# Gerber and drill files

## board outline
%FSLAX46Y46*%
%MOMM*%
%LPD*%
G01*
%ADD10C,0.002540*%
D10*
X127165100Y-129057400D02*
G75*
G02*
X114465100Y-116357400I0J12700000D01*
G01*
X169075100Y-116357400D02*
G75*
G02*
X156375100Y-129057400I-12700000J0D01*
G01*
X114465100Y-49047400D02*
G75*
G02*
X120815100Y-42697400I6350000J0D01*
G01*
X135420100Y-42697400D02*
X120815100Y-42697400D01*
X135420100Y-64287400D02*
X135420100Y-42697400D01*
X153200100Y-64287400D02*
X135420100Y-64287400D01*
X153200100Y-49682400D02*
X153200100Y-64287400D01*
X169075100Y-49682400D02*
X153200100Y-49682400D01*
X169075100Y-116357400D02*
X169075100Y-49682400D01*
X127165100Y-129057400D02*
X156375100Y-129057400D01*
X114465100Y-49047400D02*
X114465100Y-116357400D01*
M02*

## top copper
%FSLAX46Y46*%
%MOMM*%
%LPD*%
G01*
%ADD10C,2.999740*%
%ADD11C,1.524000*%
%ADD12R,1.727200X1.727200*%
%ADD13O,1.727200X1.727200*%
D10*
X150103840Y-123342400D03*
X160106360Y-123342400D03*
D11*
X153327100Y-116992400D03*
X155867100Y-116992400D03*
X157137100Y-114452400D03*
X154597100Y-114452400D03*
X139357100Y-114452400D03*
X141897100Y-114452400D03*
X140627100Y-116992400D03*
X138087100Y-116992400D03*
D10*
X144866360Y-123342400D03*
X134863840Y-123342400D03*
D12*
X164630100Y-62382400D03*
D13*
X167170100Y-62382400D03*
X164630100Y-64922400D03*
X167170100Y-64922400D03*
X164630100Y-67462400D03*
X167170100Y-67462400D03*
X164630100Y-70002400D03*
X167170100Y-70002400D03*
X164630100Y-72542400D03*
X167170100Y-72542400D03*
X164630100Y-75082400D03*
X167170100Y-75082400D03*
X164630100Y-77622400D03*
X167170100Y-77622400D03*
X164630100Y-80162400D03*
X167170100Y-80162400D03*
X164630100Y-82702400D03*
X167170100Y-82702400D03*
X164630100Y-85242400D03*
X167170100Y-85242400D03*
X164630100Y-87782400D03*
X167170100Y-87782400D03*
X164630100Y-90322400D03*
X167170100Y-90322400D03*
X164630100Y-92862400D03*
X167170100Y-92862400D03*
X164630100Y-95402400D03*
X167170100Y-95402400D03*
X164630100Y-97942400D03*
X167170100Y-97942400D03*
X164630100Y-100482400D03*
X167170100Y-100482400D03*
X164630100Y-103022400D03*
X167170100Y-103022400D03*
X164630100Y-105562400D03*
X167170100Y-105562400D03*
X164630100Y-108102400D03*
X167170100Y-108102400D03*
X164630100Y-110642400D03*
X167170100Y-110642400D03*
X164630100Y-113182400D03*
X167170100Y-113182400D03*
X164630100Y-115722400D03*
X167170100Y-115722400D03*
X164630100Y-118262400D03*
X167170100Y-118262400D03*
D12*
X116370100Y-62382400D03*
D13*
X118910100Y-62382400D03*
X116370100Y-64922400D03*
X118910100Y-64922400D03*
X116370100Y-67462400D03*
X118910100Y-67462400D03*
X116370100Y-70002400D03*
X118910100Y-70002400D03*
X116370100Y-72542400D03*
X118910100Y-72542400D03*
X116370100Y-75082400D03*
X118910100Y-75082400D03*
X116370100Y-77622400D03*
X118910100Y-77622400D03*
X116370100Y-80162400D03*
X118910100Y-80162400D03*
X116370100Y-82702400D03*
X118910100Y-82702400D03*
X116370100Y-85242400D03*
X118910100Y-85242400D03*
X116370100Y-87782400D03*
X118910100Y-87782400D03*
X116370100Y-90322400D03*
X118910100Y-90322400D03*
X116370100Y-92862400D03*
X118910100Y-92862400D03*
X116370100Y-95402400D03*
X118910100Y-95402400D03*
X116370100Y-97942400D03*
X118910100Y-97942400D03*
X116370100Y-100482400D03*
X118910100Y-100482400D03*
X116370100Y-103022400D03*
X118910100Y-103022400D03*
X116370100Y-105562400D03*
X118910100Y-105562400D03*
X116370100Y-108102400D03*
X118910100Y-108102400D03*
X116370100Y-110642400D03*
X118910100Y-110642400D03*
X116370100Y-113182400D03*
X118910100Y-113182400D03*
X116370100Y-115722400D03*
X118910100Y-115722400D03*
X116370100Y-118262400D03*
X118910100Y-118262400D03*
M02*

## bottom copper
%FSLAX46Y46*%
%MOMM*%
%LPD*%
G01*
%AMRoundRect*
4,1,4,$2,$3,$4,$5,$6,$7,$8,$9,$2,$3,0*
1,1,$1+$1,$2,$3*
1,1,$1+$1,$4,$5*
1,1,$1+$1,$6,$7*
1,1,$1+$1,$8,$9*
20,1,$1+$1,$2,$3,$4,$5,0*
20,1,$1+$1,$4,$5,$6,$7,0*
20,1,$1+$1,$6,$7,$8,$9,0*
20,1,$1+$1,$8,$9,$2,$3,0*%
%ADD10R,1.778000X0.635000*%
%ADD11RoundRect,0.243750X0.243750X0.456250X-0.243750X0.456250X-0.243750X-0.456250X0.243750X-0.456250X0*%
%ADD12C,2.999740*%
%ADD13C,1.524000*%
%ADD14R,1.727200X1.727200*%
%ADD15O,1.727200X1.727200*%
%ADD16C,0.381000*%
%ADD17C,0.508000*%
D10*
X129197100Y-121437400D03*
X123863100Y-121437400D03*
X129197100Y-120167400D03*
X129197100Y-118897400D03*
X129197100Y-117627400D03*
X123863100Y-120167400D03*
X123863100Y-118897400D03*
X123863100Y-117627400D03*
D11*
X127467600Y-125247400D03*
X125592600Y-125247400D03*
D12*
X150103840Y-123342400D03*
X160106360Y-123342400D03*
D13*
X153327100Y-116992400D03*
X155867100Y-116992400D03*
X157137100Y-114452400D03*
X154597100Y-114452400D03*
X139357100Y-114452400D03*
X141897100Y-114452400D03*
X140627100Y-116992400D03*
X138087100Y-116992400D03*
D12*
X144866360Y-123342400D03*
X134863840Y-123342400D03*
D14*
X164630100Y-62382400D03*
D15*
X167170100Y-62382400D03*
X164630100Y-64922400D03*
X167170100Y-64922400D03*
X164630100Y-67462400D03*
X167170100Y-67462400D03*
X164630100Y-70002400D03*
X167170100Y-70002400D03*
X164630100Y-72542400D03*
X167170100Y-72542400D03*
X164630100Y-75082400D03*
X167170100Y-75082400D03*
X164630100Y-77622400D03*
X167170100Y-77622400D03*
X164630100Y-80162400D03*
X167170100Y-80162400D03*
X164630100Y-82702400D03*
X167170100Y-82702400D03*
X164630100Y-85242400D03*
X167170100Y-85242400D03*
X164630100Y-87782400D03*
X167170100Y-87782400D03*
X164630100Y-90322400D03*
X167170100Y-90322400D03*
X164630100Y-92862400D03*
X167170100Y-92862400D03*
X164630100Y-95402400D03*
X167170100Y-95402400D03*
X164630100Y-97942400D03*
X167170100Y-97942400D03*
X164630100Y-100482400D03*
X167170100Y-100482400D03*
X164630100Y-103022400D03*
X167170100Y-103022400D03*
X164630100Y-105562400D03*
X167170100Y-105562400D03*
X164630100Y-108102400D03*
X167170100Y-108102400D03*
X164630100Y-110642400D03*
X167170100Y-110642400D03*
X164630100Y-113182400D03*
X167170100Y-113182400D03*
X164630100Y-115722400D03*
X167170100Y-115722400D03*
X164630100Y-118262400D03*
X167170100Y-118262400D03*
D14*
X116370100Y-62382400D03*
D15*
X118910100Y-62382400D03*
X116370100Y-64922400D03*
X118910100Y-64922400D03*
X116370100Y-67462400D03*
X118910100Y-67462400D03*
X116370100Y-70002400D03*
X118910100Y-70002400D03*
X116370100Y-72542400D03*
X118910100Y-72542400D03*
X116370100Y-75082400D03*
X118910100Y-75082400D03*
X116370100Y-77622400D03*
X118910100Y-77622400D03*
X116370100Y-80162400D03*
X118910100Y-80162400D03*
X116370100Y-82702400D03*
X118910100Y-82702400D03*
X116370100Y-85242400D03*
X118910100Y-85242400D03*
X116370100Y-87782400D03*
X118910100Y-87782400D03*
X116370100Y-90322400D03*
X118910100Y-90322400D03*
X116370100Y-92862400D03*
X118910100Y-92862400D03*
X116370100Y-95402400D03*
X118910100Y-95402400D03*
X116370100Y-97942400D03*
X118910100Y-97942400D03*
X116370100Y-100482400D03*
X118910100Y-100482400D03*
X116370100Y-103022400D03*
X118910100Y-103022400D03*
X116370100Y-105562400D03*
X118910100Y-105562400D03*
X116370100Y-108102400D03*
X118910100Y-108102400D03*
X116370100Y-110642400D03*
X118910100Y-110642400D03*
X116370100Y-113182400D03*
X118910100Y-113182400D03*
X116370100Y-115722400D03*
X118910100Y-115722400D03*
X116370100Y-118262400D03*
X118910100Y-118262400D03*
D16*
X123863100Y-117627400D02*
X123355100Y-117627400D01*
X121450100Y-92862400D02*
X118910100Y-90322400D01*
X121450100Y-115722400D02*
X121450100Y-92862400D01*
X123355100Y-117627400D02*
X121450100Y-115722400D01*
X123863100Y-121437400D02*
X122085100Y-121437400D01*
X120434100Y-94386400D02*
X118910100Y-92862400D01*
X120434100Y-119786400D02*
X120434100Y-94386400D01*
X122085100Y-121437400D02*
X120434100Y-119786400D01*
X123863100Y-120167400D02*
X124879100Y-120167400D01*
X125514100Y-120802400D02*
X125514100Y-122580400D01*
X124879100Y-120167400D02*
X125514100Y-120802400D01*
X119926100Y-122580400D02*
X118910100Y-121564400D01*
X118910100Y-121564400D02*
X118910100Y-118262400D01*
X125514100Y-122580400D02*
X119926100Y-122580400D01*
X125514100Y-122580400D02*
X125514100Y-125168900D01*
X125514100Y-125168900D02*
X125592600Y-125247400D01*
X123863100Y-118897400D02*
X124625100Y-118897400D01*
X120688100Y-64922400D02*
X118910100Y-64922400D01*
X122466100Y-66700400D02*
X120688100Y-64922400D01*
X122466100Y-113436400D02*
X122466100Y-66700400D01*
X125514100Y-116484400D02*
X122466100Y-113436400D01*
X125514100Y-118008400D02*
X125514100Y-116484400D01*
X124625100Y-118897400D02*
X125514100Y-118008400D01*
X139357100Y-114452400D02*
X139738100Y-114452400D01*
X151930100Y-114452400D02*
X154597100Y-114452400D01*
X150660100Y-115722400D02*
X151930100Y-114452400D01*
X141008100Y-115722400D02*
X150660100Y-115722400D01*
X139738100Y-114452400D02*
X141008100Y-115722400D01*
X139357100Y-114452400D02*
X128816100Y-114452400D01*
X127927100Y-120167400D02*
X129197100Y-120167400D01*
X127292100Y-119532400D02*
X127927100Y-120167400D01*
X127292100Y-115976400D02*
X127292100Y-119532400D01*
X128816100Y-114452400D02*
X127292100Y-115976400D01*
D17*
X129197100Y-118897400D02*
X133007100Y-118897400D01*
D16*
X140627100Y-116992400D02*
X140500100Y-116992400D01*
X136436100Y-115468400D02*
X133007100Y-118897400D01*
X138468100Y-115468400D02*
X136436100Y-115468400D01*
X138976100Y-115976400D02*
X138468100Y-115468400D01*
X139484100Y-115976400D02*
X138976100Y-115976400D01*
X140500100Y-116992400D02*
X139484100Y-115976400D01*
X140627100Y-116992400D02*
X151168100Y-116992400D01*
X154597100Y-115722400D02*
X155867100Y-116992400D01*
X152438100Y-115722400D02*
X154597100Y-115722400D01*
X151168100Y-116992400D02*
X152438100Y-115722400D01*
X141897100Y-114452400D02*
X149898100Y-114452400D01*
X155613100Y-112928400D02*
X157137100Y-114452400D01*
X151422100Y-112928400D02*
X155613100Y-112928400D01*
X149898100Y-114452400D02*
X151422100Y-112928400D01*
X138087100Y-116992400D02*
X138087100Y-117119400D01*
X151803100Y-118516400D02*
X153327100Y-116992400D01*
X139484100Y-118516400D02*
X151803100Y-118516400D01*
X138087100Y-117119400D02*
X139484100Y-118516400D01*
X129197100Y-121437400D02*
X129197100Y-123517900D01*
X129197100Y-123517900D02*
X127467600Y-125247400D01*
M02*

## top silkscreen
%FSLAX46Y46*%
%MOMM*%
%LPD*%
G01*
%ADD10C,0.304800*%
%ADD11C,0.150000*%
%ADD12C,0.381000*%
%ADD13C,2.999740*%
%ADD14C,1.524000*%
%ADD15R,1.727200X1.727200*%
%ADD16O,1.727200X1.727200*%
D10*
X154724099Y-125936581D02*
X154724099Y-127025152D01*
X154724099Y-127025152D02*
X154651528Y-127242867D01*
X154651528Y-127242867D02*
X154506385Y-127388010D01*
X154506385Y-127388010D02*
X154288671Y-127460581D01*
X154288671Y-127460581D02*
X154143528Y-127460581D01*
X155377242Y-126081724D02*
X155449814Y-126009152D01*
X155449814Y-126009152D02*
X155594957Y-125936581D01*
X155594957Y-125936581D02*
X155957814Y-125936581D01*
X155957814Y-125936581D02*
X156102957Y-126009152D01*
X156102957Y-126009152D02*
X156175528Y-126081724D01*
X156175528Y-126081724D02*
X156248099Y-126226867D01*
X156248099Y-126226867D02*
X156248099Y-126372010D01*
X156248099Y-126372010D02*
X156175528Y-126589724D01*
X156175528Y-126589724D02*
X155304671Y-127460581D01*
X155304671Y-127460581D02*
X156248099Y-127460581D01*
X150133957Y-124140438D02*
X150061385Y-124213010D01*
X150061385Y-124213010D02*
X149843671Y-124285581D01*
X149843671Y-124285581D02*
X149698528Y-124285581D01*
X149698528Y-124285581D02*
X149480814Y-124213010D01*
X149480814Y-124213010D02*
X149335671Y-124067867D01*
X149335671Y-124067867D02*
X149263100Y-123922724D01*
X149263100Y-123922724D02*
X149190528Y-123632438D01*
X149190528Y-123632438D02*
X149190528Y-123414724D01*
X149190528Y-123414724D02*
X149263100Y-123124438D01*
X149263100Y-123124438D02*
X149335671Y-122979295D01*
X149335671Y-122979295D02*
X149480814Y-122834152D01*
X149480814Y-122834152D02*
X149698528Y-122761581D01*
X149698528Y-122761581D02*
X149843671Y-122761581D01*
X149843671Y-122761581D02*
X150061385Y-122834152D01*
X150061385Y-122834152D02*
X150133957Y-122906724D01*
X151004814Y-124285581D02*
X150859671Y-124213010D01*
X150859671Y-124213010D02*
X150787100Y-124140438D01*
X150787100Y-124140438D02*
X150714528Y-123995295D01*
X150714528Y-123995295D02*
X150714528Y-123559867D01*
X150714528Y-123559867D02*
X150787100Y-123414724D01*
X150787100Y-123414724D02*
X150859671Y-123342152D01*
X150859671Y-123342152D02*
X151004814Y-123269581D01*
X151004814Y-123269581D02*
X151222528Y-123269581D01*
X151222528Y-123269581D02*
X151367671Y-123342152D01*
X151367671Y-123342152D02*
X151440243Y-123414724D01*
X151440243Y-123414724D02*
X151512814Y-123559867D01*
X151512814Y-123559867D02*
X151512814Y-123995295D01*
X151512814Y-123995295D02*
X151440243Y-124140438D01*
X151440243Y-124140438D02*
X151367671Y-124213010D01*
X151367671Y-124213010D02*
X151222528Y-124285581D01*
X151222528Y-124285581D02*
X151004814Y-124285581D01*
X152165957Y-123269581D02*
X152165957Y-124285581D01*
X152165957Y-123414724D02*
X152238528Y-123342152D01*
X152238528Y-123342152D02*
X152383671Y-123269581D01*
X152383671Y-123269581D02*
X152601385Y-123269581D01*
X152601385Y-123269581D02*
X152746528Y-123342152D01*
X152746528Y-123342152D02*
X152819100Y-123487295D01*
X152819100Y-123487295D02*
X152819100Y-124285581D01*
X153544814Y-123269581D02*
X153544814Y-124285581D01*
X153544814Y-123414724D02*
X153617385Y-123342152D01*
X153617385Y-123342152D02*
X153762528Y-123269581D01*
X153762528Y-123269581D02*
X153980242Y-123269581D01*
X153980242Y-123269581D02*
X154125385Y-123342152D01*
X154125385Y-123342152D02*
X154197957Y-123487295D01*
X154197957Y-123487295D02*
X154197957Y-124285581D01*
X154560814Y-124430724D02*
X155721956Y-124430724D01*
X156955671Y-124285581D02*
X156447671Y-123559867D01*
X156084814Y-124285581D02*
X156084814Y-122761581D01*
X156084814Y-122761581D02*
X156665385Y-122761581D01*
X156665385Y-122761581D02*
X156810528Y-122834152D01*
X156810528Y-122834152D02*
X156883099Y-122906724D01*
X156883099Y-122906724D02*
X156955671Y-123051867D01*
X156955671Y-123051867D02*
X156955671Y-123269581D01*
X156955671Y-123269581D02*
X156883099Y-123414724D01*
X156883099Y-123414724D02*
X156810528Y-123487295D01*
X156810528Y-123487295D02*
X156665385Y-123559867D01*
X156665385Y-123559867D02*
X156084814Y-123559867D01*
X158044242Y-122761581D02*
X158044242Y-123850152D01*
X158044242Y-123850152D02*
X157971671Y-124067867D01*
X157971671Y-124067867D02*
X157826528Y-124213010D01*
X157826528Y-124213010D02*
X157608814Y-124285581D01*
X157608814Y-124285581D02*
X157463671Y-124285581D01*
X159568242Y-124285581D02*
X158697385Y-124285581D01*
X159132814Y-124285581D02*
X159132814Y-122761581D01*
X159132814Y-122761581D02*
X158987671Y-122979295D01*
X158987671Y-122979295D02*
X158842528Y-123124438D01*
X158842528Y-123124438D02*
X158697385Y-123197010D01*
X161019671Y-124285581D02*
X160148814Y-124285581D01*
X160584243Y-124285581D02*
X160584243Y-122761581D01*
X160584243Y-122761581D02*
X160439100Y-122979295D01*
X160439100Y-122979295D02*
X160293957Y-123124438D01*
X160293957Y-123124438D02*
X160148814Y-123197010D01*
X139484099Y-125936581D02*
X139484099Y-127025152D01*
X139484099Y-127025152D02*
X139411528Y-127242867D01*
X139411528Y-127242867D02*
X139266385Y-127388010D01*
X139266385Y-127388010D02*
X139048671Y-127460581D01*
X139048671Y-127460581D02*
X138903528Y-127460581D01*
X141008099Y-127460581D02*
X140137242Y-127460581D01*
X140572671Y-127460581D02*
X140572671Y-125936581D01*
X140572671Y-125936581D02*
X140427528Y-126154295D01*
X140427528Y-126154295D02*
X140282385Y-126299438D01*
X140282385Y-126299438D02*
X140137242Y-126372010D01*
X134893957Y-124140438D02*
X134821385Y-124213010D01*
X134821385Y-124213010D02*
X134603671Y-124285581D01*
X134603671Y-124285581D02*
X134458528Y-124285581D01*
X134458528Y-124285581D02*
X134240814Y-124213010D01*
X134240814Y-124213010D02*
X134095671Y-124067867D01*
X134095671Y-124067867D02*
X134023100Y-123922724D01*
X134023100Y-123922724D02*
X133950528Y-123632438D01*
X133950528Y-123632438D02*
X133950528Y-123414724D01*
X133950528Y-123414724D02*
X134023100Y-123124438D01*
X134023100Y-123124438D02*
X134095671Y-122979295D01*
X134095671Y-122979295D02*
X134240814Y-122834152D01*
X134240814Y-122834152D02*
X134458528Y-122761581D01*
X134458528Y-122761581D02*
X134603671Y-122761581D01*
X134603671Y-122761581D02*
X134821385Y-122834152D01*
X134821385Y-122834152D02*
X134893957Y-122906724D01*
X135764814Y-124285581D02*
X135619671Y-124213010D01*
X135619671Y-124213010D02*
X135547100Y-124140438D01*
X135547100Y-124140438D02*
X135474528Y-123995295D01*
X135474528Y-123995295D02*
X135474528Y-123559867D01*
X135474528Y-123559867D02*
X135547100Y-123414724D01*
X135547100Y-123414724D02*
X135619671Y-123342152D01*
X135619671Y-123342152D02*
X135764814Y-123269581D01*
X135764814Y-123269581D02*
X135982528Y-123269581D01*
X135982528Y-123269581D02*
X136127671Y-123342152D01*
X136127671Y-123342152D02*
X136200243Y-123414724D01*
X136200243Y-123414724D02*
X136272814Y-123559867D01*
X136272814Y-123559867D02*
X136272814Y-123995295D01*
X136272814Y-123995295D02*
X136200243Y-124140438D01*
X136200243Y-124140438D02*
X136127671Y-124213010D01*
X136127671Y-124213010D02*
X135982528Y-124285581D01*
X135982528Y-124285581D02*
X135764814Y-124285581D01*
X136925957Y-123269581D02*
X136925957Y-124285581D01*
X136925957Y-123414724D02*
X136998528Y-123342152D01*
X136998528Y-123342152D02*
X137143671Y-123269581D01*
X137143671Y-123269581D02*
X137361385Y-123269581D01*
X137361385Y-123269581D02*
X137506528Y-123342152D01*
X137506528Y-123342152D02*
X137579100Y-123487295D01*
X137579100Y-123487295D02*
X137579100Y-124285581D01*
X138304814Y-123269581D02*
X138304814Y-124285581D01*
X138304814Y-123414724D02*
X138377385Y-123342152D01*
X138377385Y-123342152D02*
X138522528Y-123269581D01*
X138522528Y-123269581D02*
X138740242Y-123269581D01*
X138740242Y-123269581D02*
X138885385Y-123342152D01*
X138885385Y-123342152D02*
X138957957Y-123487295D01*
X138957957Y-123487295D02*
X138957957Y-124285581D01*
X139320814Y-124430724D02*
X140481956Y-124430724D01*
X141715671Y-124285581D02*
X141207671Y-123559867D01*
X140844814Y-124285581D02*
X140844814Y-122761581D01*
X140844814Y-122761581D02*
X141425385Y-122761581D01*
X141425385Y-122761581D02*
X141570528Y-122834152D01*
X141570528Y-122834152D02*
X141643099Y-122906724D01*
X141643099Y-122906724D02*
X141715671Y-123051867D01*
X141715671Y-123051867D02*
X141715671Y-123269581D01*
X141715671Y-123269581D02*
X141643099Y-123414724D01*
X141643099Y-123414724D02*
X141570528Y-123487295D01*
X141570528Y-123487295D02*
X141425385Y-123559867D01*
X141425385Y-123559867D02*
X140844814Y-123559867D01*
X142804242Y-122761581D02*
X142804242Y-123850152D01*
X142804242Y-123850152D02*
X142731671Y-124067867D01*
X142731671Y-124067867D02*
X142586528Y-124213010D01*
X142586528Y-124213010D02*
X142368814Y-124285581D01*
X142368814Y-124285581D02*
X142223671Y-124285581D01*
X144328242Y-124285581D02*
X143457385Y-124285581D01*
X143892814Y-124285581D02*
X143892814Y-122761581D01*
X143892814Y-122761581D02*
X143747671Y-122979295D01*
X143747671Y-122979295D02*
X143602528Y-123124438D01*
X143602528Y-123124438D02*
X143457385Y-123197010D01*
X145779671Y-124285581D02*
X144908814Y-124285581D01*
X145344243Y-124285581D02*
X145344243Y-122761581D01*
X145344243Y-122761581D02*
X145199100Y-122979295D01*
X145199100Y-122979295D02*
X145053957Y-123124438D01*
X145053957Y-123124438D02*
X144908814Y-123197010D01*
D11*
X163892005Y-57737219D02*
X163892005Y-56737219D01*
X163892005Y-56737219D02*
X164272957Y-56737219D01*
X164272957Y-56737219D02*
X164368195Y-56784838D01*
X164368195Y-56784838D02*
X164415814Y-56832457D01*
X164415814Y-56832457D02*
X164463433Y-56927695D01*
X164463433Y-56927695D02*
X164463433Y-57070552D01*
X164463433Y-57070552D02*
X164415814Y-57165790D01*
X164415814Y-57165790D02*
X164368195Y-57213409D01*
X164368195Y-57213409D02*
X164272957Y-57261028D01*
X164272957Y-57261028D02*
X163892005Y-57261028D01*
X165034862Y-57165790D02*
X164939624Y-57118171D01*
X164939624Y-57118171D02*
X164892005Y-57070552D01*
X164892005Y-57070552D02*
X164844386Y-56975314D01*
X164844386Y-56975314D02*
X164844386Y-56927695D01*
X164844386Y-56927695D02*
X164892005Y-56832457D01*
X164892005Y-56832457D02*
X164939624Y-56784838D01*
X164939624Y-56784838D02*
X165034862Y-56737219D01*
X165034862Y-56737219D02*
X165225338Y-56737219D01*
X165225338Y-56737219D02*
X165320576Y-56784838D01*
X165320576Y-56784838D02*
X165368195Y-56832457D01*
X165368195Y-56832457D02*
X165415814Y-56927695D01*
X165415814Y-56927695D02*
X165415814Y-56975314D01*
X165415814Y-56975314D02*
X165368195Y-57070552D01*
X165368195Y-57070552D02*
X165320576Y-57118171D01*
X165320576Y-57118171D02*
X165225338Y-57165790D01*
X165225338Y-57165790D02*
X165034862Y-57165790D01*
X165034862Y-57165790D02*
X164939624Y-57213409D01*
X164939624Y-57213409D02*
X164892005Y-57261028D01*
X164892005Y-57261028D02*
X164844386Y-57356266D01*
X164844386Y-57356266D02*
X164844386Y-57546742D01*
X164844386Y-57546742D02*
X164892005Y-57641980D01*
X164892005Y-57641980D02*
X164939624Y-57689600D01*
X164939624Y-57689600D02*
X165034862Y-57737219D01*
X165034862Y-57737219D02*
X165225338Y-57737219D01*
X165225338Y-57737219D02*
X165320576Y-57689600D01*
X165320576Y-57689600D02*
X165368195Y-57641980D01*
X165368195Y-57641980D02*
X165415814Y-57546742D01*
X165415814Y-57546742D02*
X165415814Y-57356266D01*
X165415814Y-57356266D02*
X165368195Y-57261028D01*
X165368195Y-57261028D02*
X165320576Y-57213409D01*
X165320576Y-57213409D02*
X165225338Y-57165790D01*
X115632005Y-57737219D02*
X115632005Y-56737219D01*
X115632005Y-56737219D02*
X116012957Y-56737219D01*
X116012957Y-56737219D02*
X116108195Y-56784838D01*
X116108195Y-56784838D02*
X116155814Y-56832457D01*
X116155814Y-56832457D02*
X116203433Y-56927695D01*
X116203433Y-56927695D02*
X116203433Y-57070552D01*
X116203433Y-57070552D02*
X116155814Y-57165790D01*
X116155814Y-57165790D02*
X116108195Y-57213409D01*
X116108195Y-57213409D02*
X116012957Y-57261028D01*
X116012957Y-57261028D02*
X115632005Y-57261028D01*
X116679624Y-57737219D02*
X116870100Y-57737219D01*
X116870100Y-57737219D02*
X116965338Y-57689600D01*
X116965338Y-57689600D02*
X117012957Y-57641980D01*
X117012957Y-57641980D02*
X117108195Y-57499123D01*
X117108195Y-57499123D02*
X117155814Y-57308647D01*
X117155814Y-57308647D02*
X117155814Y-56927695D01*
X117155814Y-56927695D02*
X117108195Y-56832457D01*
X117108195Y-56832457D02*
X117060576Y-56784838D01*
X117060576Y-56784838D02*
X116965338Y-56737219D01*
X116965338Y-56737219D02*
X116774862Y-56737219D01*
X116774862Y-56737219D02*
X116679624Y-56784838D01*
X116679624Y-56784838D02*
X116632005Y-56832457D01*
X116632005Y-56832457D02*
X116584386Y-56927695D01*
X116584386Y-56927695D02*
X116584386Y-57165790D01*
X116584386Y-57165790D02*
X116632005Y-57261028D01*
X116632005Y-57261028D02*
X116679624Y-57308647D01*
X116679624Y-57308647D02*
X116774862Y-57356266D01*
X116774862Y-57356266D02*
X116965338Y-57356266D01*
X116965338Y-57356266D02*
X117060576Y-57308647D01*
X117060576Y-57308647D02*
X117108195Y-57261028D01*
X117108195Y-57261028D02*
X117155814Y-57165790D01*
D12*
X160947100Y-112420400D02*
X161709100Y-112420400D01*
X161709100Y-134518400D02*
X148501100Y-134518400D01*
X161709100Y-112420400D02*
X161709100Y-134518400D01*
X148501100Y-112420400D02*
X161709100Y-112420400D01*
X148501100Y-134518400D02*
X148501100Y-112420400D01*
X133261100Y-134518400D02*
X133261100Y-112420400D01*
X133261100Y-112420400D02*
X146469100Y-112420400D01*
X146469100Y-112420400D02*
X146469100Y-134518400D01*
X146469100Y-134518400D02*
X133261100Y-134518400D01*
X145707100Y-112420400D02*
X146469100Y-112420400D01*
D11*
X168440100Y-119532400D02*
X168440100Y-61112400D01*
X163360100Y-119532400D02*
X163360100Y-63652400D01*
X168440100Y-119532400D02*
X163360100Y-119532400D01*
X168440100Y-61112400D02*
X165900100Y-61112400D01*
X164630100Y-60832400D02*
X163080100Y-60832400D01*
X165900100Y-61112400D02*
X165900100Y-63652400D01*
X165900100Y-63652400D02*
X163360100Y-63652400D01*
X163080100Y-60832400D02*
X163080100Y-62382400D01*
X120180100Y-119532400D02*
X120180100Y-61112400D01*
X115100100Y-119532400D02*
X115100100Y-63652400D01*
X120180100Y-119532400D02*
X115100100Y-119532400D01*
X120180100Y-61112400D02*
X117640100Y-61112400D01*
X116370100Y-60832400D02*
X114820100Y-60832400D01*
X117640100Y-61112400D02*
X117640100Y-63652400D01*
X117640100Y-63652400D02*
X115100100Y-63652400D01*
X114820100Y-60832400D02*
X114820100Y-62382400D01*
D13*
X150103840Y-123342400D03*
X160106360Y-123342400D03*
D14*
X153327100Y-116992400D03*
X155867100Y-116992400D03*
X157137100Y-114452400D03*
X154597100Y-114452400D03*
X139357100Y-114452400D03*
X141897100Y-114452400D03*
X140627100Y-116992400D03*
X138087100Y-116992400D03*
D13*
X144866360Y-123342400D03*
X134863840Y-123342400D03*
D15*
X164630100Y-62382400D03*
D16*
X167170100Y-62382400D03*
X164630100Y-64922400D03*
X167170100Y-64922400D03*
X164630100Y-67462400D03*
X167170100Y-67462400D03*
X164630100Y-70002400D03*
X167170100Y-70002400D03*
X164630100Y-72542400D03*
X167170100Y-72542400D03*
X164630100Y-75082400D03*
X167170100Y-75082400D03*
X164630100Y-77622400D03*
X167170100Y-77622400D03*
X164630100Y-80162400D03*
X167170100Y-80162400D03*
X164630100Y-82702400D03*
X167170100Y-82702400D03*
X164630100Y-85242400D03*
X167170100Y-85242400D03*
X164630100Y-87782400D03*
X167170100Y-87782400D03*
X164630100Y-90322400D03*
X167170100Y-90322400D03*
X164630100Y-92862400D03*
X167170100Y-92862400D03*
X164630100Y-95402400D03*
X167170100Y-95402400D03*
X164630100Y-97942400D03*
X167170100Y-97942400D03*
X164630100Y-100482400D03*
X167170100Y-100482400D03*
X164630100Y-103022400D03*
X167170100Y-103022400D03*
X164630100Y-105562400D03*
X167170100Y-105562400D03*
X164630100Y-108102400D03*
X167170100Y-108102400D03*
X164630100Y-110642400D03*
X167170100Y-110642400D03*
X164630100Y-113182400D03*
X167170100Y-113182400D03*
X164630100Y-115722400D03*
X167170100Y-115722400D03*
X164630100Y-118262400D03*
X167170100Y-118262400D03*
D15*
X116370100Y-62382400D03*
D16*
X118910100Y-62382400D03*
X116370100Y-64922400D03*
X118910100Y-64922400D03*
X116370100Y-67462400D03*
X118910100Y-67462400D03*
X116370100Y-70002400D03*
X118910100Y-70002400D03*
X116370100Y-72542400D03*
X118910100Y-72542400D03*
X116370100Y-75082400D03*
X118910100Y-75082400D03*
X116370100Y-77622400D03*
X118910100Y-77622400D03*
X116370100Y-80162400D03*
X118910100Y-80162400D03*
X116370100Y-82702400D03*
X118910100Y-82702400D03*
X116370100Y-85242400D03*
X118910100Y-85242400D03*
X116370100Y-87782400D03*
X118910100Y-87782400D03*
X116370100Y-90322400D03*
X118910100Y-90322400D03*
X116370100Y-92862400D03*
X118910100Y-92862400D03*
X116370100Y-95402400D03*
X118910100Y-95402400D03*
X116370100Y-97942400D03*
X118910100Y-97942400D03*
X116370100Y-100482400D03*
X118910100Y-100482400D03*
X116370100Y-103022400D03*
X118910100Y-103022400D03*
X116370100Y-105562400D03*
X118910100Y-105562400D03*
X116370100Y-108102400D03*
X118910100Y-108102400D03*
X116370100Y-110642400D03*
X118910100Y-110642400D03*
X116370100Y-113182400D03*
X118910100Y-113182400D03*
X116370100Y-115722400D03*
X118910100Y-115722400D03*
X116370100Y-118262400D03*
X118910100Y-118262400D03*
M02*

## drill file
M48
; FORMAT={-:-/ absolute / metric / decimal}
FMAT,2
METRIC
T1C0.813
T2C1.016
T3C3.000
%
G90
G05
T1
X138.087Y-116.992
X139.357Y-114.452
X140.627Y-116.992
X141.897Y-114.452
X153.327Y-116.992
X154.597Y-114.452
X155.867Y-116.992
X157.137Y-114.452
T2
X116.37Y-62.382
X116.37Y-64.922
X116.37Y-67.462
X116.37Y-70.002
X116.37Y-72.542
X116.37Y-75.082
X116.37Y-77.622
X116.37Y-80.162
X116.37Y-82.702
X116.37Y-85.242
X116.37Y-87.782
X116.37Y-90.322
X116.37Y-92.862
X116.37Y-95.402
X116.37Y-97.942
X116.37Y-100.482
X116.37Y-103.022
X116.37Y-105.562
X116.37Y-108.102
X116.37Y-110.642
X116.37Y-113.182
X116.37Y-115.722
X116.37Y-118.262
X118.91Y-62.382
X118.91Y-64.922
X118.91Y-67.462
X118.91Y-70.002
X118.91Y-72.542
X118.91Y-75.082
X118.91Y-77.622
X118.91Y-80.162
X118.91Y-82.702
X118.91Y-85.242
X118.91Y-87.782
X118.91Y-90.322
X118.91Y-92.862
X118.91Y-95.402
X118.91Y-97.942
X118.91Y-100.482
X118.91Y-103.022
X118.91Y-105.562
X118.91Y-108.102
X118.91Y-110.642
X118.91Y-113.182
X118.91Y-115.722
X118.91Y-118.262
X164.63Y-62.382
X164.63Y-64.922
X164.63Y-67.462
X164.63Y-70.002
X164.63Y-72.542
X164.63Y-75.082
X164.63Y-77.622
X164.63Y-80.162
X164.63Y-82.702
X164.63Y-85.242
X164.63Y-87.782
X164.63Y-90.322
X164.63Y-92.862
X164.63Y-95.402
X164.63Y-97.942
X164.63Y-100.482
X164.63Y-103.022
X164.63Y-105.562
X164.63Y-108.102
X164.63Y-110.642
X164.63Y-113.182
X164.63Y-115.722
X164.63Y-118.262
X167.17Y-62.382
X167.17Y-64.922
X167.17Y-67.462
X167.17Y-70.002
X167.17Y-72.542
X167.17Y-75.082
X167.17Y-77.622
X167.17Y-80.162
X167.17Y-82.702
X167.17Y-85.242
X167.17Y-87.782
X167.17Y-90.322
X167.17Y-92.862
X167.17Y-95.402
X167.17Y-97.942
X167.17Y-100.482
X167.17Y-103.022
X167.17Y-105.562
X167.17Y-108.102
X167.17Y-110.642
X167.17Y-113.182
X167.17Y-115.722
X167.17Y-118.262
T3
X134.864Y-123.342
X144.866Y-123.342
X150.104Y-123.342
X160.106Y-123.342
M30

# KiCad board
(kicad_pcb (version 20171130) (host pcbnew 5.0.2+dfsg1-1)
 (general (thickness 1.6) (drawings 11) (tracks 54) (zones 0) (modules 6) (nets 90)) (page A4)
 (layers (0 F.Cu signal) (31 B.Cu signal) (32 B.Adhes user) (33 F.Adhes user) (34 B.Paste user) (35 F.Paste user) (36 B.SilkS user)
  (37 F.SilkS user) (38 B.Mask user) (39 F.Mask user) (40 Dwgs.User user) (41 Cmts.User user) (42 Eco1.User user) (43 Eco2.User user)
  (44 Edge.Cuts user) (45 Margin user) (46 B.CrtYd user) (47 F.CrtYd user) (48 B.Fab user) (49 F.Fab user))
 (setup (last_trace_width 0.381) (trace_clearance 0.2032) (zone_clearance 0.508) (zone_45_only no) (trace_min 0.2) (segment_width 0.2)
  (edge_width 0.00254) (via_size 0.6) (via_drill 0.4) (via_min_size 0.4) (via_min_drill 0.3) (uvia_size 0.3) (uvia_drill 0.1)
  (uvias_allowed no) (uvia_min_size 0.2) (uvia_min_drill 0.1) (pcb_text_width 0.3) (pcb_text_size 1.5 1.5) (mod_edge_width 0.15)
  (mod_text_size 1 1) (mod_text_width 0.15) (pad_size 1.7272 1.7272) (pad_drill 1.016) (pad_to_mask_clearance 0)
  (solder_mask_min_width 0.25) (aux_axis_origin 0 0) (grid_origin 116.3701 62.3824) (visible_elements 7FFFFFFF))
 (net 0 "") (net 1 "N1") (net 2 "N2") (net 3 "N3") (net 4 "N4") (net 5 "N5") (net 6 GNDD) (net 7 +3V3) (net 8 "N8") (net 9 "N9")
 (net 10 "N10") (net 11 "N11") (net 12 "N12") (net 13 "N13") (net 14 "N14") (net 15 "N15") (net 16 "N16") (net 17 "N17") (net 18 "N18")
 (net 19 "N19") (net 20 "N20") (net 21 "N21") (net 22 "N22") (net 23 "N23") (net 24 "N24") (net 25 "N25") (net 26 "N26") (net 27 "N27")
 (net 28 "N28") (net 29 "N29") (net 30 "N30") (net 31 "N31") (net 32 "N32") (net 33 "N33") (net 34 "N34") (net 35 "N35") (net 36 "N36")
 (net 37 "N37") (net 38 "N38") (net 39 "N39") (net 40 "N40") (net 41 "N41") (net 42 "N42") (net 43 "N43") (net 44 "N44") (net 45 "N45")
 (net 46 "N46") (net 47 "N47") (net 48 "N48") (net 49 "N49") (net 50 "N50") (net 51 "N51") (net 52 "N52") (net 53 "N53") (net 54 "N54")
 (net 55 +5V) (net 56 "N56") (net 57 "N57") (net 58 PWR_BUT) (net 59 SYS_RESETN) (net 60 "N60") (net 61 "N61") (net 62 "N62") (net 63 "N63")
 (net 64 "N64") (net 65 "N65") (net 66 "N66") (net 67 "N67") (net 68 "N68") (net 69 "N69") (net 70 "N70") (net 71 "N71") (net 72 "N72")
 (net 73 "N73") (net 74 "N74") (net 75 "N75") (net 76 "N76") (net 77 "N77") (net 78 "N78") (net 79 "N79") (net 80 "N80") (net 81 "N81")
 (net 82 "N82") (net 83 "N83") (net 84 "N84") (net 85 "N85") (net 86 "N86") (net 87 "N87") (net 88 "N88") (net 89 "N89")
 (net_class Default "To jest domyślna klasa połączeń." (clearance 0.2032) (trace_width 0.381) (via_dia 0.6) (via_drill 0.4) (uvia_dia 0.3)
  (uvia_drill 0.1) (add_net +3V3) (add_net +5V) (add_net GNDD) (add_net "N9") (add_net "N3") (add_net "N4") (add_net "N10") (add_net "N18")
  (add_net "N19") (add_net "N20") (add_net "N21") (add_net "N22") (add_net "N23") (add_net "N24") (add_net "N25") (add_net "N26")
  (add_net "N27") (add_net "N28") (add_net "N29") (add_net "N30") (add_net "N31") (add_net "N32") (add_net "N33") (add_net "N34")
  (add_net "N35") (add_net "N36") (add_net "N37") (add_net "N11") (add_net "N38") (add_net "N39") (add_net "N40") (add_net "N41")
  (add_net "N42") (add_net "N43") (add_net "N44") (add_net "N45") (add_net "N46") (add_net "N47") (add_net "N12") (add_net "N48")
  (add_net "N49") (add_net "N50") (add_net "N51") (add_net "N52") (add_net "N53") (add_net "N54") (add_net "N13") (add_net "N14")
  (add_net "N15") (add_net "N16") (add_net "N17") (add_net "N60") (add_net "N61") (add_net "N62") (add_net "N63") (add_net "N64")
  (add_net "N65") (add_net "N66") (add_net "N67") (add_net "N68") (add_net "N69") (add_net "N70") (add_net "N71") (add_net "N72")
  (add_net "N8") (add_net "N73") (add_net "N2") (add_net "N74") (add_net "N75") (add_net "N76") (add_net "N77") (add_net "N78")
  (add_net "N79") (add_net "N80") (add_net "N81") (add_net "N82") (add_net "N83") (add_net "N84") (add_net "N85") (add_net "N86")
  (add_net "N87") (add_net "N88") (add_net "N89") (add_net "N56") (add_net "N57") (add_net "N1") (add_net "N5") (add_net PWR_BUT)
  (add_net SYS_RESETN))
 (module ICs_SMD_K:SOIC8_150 (layer B.Cu) (at 126.5301 119.5324 90)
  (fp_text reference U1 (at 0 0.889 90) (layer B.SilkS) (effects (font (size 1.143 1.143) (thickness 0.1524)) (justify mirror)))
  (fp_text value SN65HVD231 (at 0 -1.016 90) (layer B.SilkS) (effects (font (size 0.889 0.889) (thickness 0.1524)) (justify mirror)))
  (pad 8 smd rect (at -1.905 2.667 90) (size 0.635 1.778) (layers B.Cu B.Paste B.Mask) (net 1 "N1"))
  (pad 1 smd rect (at -1.905 -2.667 90) (size 0.635 1.778) (layers B.Cu B.Paste B.Mask) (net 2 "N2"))
  (pad 7 smd rect (at -0.635 2.667 90) (size 0.635 1.778) (layers B.Cu B.Paste B.Mask) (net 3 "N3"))
  (pad 6 smd rect (at 0.635 2.667 90) (size 0.635 1.778) (layers B.Cu B.Paste B.Mask) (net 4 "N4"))
  (pad 5 smd rect (at 1.905 2.667 90) (size 0.635 1.778) (layers B.Cu B.Paste B.Mask) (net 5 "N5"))
  (pad 2 smd rect (at -0.635 -2.667 90) (size 0.635 1.778) (layers B.Cu B.Paste B.Mask) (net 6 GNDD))
  (pad 3 smd rect (at 0.635 -2.667 90) (size 0.635 1.778) (layers B.Cu B.Paste B.Mask) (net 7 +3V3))
  (pad 4 smd rect (at 1.905 -2.667 90) (size 0.635 1.778) (layers B.Cu B.Paste B.Mask) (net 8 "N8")))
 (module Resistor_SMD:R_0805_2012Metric (layer B.Cu) (at 126.5301 125.2474 180)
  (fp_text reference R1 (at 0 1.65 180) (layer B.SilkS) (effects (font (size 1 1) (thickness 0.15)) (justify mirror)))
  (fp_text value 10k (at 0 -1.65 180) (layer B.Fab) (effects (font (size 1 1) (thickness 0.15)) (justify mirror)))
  (pad 1 smd roundrect (at -0.9375 0 180) (size 0.975 1.4) (layers B.Cu B.Paste B.Mask) (roundrect_rratio 0.25) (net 1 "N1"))
  (pad 2 smd roundrect (at 0.9375 0 180) (size 0.975 1.4) (layers B.Cu B.Paste B.Mask) (roundrect_rratio 0.25) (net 6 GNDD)))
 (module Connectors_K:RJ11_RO (layer F.Cu) (at 155.1051 123.3424)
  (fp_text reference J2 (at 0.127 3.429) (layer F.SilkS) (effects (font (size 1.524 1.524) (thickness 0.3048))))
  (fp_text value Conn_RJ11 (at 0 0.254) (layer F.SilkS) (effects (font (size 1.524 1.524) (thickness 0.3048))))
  (fp_line (start 5.842 -10.922) (end 6.604 -10.922) (layer F.SilkS) (width 0.381))
  (fp_line (start 6.604 11.176) (end -6.604 11.176) (layer F.SilkS) (width 0.381))
  (fp_line (start 6.604 -10.922) (end 6.604 11.176) (layer F.SilkS) (width 0.381))
  (fp_line (start -6.604 -10.922) (end 6.604 -10.922) (layer F.SilkS) (width 0.381))
  (fp_line (start -6.604 11.176) (end -6.604 -10.922) (layer F.SilkS) (width 0.381))
  (pad 7 thru_hole circle (at -5.00126 0) (size 2.99974 2.99974) (drill 2.99974) (layers *.Cu *.Mask F.SilkS))
  (pad 8 thru_hole circle (at 5.00126 0) (size 2.99974 2.99974) (drill 2.99974) (layers *.Cu *.Mask F.SilkS))
  (pad 2 thru_hole circle (at -1.778 -6.35) (size 1.524 1.524) (drill 0.8128) (layers *.Cu *.Mask F.SilkS) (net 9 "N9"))
  (pad 4 thru_hole circle (at 0.762 -6.35) (size 1.524 1.524) (drill 0.8128) (layers *.Cu *.Mask F.SilkS) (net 4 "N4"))
  (pad 5 thru_hole circle (at 2.032 -8.89) (size 1.524 1.524) (drill 0.8128) (layers *.Cu *.Mask F.SilkS) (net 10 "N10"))
  (pad 3 thru_hole circle (at -0.508 -8.89) (size 1.524 1.524) (drill 0.8128) (layers *.Cu *.Mask F.SilkS) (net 3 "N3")))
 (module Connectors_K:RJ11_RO (layer F.Cu) (at 139.8651 123.3424)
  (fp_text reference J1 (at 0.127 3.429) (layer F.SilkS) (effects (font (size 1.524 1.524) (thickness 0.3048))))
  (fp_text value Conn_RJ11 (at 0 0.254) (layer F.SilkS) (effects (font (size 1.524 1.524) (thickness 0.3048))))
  (fp_line (start -6.604 11.176) (end -6.604 -10.922) (layer F.SilkS) (width 0.381))
  (fp_line (start -6.604 -10.922) (end 6.604 -10.922) (layer F.SilkS) (width 0.381))
  (fp_line (start 6.604 -10.922) (end 6.604 11.176) (layer F.SilkS) (width 0.381))
  (fp_line (start 6.604 11.176) (end -6.604 11.176) (layer F.SilkS) (width 0.381))
  (fp_line (start 5.842 -10.922) (end 6.604 -10.922) (layer F.SilkS) (width 0.381))
  (pad 3 thru_hole circle (at -0.508 -8.89) (size 1.524 1.524) (drill 0.8128) (layers *.Cu *.Mask F.SilkS) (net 3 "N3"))
  (pad 5 thru_hole circle (at 2.032 -8.89) (size 1.524 1.524) (drill 0.8128) (layers *.Cu *.Mask F.SilkS) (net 10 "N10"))
  (pad 4 thru_hole circle (at 0.762 -6.35) (size 1.524 1.524) (drill 0.8128) (layers *.Cu *.Mask F.SilkS) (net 4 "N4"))
  (pad 2 thru_hole circle (at -1.778 -6.35) (size 1.524 1.524) (drill 0.8128) (layers *.Cu *.Mask F.SilkS) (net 9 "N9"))
  (pad 8 thru_hole circle (at 5.00126 0) (size 2.99974 2.99974) (drill 2.99974) (layers *.Cu *.Mask F.SilkS))
  (pad 7 thru_hole circle (at -5.00126 0) (size 2.99974 2.99974) (drill 2.99974) (layers *.Cu *.Mask F.SilkS)))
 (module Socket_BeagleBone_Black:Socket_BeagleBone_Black (layer F.Cu) (at 164.6301 62.3824)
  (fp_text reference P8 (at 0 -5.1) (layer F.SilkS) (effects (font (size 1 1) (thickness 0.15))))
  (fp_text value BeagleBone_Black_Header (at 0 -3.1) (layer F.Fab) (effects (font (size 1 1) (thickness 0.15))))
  (fp_line (start 3.81 57.15) (end 3.81 -1.27) (layer F.SilkS) (width 0.15))
  (fp_line (start -1.27 57.15) (end -1.27 1.27) (layer F.SilkS) (width 0.15))
  (fp_line (start 3.81 57.15) (end -1.27 57.15) (layer F.SilkS) (width 0.15))
  (fp_line (start 3.81 -1.27) (end 1.27 -1.27) (layer F.SilkS) (width 0.15))
  (fp_line (start 0 -1.55) (end -1.55 -1.55) (layer F.SilkS) (width 0.15))
  (fp_line (start 1.27 -1.27) (end 1.27 1.27) (layer F.SilkS) (width 0.15))
  (fp_line (start 1.27 1.27) (end -1.27 1.27) (layer F.SilkS) (width 0.15))
  (fp_line (start -1.55 -1.55) (end -1.55 0) (layer F.SilkS) (width 0.15))
  (pad 1 thru_hole rect (at 0 0) (size 1.7272 1.7272) (drill 1.016) (layers *.Cu *.Mask F.SilkS) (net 6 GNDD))
  (pad 2 thru_hole oval (at 2.54 0) (size 1.7272 1.7272) (drill 1.016) (layers *.Cu *.Mask F.SilkS) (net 6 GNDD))
  (pad 3 thru_hole oval (at 0 2.54) (size 1.7272 1.7272) (drill 1.016) (layers *.Cu *.Mask F.SilkS) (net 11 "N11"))
  (pad 4 thru_hole oval (at 2.54 2.54) (size 1.7272 1.7272) (drill 1.016) (layers *.Cu *.Mask F.SilkS) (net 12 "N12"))
  (pad 5 thru_hole oval (at 0 5.08) (size 1.7272 1.7272) (drill 1.016) (layers *.Cu *.Mask F.SilkS) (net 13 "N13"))
  (pad 6 thru_hole oval (at 2.54 5.08) (size 1.7272 1.7272) (drill 1.016) (layers *.Cu *.Mask F.SilkS) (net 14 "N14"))
  (pad 7 thru_hole oval (at 0 7.62) (size 1.7272 1.7272) (drill 1.016) (layers *.Cu *.Mask F.SilkS) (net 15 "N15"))
  (pad 8 thru_hole oval (at 2.54 7.62) (size 1.7272 1.7272) (drill 1.016) (layers *.Cu *.Mask F.SilkS) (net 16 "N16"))
  (pad 9 thru_hole oval (at 0 10.16) (size 1.7272 1.7272) (drill 1.016) (layers *.Cu *.Mask F.SilkS) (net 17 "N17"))
  (pad 10 thru_hole oval (at 2.54 10.16) (size 1.7272 1.7272) (drill 1.016) (layers *.Cu *.Mask F.SilkS) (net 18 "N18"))
  (pad 11 thru_hole oval (at 0 12.7) (size 1.7272 1.7272) (drill 1.016) (layers *.Cu *.Mask F.SilkS) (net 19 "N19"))
  (pad 12 thru_hole oval (at 2.54 12.7) (size 1.7272 1.7272) (drill 1.016) (layers *.Cu *.Mask F.SilkS) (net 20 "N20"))
  (pad 13 thru_hole oval (at 0 15.24) (size 1.7272 1.7272) (drill 1.016) (layers *.Cu *.Mask F.SilkS) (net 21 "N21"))
  (pad 14 thru_hole oval (at 2.54 15.24) (size 1.7272 1.7272) (drill 1.016) (layers *.Cu *.Mask F.SilkS) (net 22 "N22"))
  (pad 15 thru_hole oval (at 0 17.78) (size 1.7272 1.7272) (drill 1.016) (layers *.Cu *.Mask F.SilkS) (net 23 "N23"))
  (pad 16 thru_hole oval (at 2.54 17.78) (size 1.7272 1.7272) (drill 1.016) (layers *.Cu *.Mask F.SilkS) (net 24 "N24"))
  (pad 17 thru_hole oval (at 0 20.32) (size 1.7272 1.7272) (drill 1.016) (layers *.Cu *.Mask F.SilkS) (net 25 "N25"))
  (pad 18 thru_hole oval (at 2.54 20.32) (size 1.7272 1.7272) (drill 1.016) (layers *.Cu *.Mask F.SilkS) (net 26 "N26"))
  (pad 19 thru_hole oval (at 0 22.86) (size 1.7272 1.7272) (drill 1.016) (layers *.Cu *.Mask F.SilkS) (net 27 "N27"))
  (pad 20 thru_hole oval (at 2.54 22.86) (size 1.7272 1.7272) (drill 1.016) (layers *.Cu *.Mask F.SilkS) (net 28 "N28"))
  (pad 21 thru_hole oval (at 0 25.4) (size 1.7272 1.7272) (drill 1.016) (layers *.Cu *.Mask F.SilkS) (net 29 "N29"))
  (pad 22 thru_hole oval (at 2.54 25.4) (size 1.7272 1.7272) (drill 1.016) (layers *.Cu *.Mask F.SilkS) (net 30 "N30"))
  (pad 23 thru_hole oval (at 0 27.94) (size 1.7272 1.7272) (drill 1.016) (layers *.Cu *.Mask F.SilkS) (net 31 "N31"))
  (pad 24 thru_hole oval (at 2.54 27.94) (size 1.7272 1.7272) (drill 1.016) (layers *.Cu *.Mask F.SilkS) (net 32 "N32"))
  (pad 25 thru_hole oval (at 0 30.48) (size 1.7272 1.7272) (drill 1.016) (layers *.Cu *.Mask F.SilkS) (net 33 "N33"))
  (pad 26 thru_hole oval (at 2.54 30.48) (size 1.7272 1.7272) (drill 1.016) (layers *.Cu *.Mask F.SilkS) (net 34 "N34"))
  (pad 27 thru_hole oval (at 0 33.02) (size 1.7272 1.7272) (drill 1.016) (layers *.Cu *.Mask F.SilkS) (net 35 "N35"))
  (pad 28 thru_hole oval (at 2.54 33.02) (size 1.7272 1.7272) (drill 1.016) (layers *.Cu *.Mask F.SilkS) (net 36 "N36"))
  (pad 29 thru_hole oval (at 0 35.56) (size 1.7272 1.7272) (drill 1.016) (layers *.Cu *.Mask F.SilkS) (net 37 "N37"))
  (pad 30 thru_hole oval (at 2.54 35.56) (size 1.7272 1.7272) (drill 1.016) (layers *.Cu *.Mask F.SilkS) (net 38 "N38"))
  (pad 31 thru_hole oval (at 0 38.1) (size 1.7272 1.7272) (drill 1.016) (layers *.Cu *.Mask F.SilkS) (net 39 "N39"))
  (pad 32 thru_hole oval (at 2.54 38.1) (size 1.7272 1.7272) (drill 1.016) (layers *.Cu *.Mask F.SilkS) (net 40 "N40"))
  (pad 33 thru_hole oval (at 0 40.64) (size 1.7272 1.7272) (drill 1.016) (layers *.Cu *.Mask F.SilkS) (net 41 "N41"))
  (pad 34 thru_hole oval (at 2.54 40.64) (size 1.7272 1.7272) (drill 1.016) (layers *.Cu *.Mask F.SilkS) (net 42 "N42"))
  (pad 35 thru_hole oval (at 0 43.18) (size 1.7272 1.7272) (drill 1.016) (layers *.Cu *.Mask F.SilkS) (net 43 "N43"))
  (pad 36 thru_hole oval (at 2.54 43.18) (size 1.7272 1.7272) (drill 1.016) (layers *.Cu *.Mask F.SilkS) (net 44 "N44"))
  (pad 37 thru_hole oval (at 0 45.72) (size 1.7272 1.7272) (drill 1.016) (layers *.Cu *.Mask F.SilkS) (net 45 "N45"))
  (pad 38 thru_hole oval (at 2.54 45.72) (size 1.7272 1.7272) (drill 1.016) (layers *.Cu *.Mask F.SilkS) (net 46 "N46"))
  (pad 39 thru_hole oval (at 0 48.26) (size 1.7272 1.7272) (drill 1.016) (layers *.Cu *.Mask F.SilkS) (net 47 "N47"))
  (pad 40 thru_hole oval (at 2.54 48.26) (size 1.7272 1.7272) (drill 1.016) (layers *.Cu *.Mask F.SilkS) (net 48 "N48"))
  (pad 41 thru_hole oval (at 0 50.8) (size 1.7272 1.7272) (drill 1.016) (layers *.Cu *.Mask F.SilkS) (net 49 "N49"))
  (pad 42 thru_hole oval (at 2.54 50.8) (size 1.7272 1.7272) (drill 1.016) (layers *.Cu *.Mask F.SilkS) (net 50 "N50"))
  (pad 43 thru_hole oval (at 0 53.34) (size 1.7272 1.7272) (drill 1.016) (layers *.Cu *.Mask F.SilkS) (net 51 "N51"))
  (pad 44 thru_hole oval (at 2.54 53.34) (size 1.7272 1.7272) (drill 1.016) (layers *.Cu *.Mask F.SilkS) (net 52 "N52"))
  (pad 45 thru_hole oval (at 0 55.88) (size 1.7272 1.7272) (drill 1.016) (layers *.Cu *.Mask F.SilkS) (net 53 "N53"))
  (pad 46 thru_hole oval (at 2.54 55.88) (size 1.7272 1.7272) (drill 1.016) (layers *.Cu *.Mask F.SilkS) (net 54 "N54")))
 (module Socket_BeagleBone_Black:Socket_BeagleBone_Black (layer F.Cu) (at 116.3701 62.3824)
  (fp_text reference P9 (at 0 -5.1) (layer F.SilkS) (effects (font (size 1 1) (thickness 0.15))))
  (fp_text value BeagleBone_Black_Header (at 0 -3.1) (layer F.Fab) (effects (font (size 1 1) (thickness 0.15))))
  (fp_line (start 3.81 57.15) (end 3.81 -1.27) (layer F.SilkS) (width 0.15))
  (fp_line (start -1.27 57.15) (end -1.27 1.27) (layer F.SilkS) (width 0.15))
  (fp_line (start 3.81 57.15) (end -1.27 57.15) (layer F.SilkS) (width 0.15))
  (fp_line (start 3.81 -1.27) (end 1.27 -1.27) (layer F.SilkS) (width 0.15))
  (fp_line (start 0 -1.55) (end -1.55 -1.55) (layer F.SilkS) (width 0.15))
  (fp_line (start 1.27 -1.27) (end 1.27 1.27) (layer F.SilkS) (width 0.15))
  (fp_line (start 1.27 1.27) (end -1.27 1.27) (layer F.SilkS) (width 0.15))
  (fp_line (start -1.55 -1.55) (end -1.55 0) (layer F.SilkS) (width 0.15))
  (pad 1 thru_hole rect (at 0 0) (size 1.7272 1.7272) (drill 1.016) (layers *.Cu *.Mask F.SilkS) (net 6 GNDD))
  (pad 2 thru_hole oval (at 2.54 0) (size 1.7272 1.7272) (drill 1.016) (layers *.Cu *.Mask F.SilkS) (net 6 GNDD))
  (pad 3 thru_hole oval (at 0 2.54) (size 1.7272 1.7272) (drill 1.016) (layers *.Cu *.Mask F.SilkS) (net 7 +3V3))
  (pad 4 thru_hole oval (at 2.54 2.54) (size 1.7272 1.7272) (drill 1.016) (layers *.Cu *.Mask F.SilkS) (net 7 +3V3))
  (pad 5 thru_hole oval (at 0 5.08) (size 1.7272 1.7272) (drill 1.016) (layers *.Cu *.Mask F.SilkS) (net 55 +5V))
  (pad 6 thru_hole oval (at 2.54 5.08) (size 1.7272 1.7272) (drill 1.016) (layers *.Cu *.Mask F.SilkS) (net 55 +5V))
  (pad 7 thru_hole oval (at 0 7.62) (size 1.7272 1.7272) (drill 1.016) (layers *.Cu *.Mask F.SilkS) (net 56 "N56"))
  (pad 8 thru_hole oval (at 2.54 7.62) (size 1.7272 1.7272) (drill 1.016) (layers *.Cu *.Mask F.SilkS) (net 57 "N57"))
  (pad 9 thru_hole oval (at 0 10.16) (size 1.7272 1.7272) (drill 1.016) (layers *.Cu *.Mask F.SilkS) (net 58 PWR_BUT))
  (pad 10 thru_hole oval (at 2.54 10.16) (size 1.7272 1.7272) (drill 1.016) (layers *.Cu *.Mask F.SilkS) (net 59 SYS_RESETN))
  (pad 11 thru_hole oval (at 0 12.7) (size 1.7272 1.7272) (drill 1.016) (layers *.Cu *.Mask F.SilkS) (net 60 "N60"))
  (pad 12 thru_hole oval (at 2.54 12.7) (size 1.7272 1.7272) (drill 1.016) (layers *.Cu *.Mask F.SilkS) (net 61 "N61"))
  (pad 13 thru_hole oval (at 0 15.24) (size 1.7272 1.7272) (drill 1.016) (layers *.Cu *.Mask F.SilkS) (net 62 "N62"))
  (pad 14 thru_hole oval (at 2.54 15.24) (size 1.7272 1.7272) (drill 1.016) (layers *.Cu *.Mask F.SilkS) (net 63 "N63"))
  (pad 15 thru_hole oval (at 0 17.78) (size 1.7272 1.7272) (drill 1.016) (layers *.Cu *.Mask F.SilkS) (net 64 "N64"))
  (pad 16 thru_hole oval (at 2.54 17.78) (size 1.7272 1.7272) (drill 1.016) (layers *.Cu *.Mask F.SilkS) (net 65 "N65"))
  (pad 17 thru_hole oval (at 0 20.32) (size 1.7272 1.7272) (drill 1.016) (layers *.Cu *.Mask F.SilkS) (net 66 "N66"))
  (pad 18 thru_hole oval (at 2.54 20.32) (size 1.7272 1.7272) (drill 1.016) (layers *.Cu *.Mask F.SilkS) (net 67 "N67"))
  (pad 19 thru_hole oval (at 0 22.86) (size 1.7272 1.7272) (drill 1.016) (layers *.Cu *.Mask F.SilkS) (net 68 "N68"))
  (pad 20 thru_hole oval (at 2.54 22.86) (size 1.7272 1.7272) (drill 1.016) (layers *.Cu *.Mask F.SilkS) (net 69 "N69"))
  (pad 21 thru_hole oval (at 0 25.4) (size 1.7272 1.7272) (drill 1.016) (layers *.Cu *.Mask F.SilkS) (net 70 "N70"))
  (pad 22 thru_hole oval (at 2.54 25.4) (size 1.7272 1.7272) (drill 1.016) (layers *.Cu *.Mask F.SilkS) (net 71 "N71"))
  (pad 23 thru_hole oval (at 0 27.94) (size 1.7272 1.7272) (drill 1.016) (layers *.Cu *.Mask F.SilkS) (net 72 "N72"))
  (pad 24 thru_hole oval (at 2.54 27.94) (size 1.7272 1.7272) (drill 1.016) (layers *.Cu *.Mask F.SilkS) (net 8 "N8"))
  (pad 25 thru_hole oval (at 0 30.48) (size 1.7272 1.7272) (drill 1.016) (layers *.Cu *.Mask F.SilkS) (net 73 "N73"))
  (pad 26 thru_hole oval (at 2.54 30.48) (size 1.7272 1.7272) (drill 1.016) (layers *.Cu *.Mask F.SilkS) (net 2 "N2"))
  (pad 27 thru_hole oval (at 0 33.02) (size 1.7272 1.7272) (drill 1.016) (layers *.Cu *.Mask F.SilkS) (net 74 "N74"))
  (pad 28 thru_hole oval (at 2.54 33.02) (size 1.7272 1.7272) (drill 1.016) (layers *.Cu *.Mask F.SilkS) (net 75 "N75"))
  (pad 29 thru_hole oval (at 0 35.56) (size 1.7272 1.7272) (drill 1.016) (layers *.Cu *.Mask F.SilkS) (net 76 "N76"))
  (pad 30 thru_hole oval (at 2.54 35.56) (size 1.7272 1.7272) (drill 1.016) (layers *.Cu *.Mask F.SilkS) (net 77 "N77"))
  (pad 31 thru_hole oval (at 0 38.1) (size 1.7272 1.7272) (drill 1.016) (layers *.Cu *.Mask F.SilkS) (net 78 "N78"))
  (pad 32 thru_hole oval (at 2.54 38.1) (size 1.7272 1.7272) (drill 1.016) (layers *.Cu *.Mask F.SilkS) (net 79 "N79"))
  (pad 33 thru_hole oval (at 0 40.64) (size 1.7272 1.7272) (drill 1.016) (layers *.Cu *.Mask F.SilkS) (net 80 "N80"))
  (pad 34 thru_hole oval (at 2.54 40.64) (size 1.7272 1.7272) (drill 1.016) (layers *.Cu *.Mask F.SilkS) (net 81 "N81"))
  (pad 35 thru_hole oval (at 0 43.18) (size 1.7272 1.7272) (drill 1.016) (layers *.Cu *.Mask F.SilkS) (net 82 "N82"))
  (pad 36 thru_hole oval (at 2.54 43.18) (size 1.7272 1.7272) (drill 1.016) (layers *.Cu *.Mask F.SilkS) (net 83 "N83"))
  (pad 37 thru_hole oval (at 0 45.72) (size 1.7272 1.7272) (drill 1.016) (layers *.Cu *.Mask F.SilkS) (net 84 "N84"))
  (pad 38 thru_hole oval (at 2.54 45.72) (size 1.7272 1.7272) (drill 1.016) (layers *.Cu *.Mask F.SilkS) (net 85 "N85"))
  (pad 39 thru_hole oval (at 0 48.26) (size 1.7272 1.7272) (drill 1.016) (layers *.Cu *.Mask F.SilkS) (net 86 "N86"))
  (pad 40 thru_hole oval (at 2.54 48.26) (size 1.7272 1.7272) (drill 1.016) (layers *.Cu *.Mask F.SilkS) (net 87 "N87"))
  (pad 41 thru_hole oval (at 0 50.8) (size 1.7272 1.7272) (drill 1.016) (layers *.Cu *.Mask F.SilkS) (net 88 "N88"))
  (pad 42 thru_hole oval (at 2.54 50.8) (size 1.7272 1.7272) (drill 1.016) (layers *.Cu *.Mask F.SilkS) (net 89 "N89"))
  (pad 43 thru_hole oval (at 0 53.34) (size 1.7272 1.7272) (drill 1.016) (layers *.Cu *.Mask F.SilkS) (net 6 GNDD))
  (pad 44 thru_hole oval (at 2.54 53.34) (size 1.7272 1.7272) (drill 1.016) (layers *.Cu *.Mask F.SilkS) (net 6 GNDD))
  (pad 45 thru_hole oval (at 0 55.88) (size 1.7272 1.7272) (drill 1.016) (layers *.Cu *.Mask F.SilkS) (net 6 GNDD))
  (pad 46 thru_hole oval (at 2.54 55.88) (size 1.7272 1.7272) (drill 1.016) (layers *.Cu *.Mask F.SilkS) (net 6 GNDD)))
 (gr_arc (start 127.1651 116.3574) (end 127.1651 129.0574) (angle 90) (layer Edge.Cuts) (width 0.00254))
 (gr_arc (start 156.3751 116.3574) (end 169.0751 116.3574) (angle 90) (layer Edge.Cuts) (width 0.00254))
 (gr_arc (start 120.8151 49.0474) (end 114.4651 49.0474) (angle 90) (layer Edge.Cuts) (width 0.00254))
 (gr_line (start 135.4201 42.6974) (end 120.8151 42.6974) (layer Edge.Cuts) (width 0.00254))
 (gr_line (start 135.4201 64.2874) (end 135.4201 42.6974) (layer Edge.Cuts) (width 0.00254))
 (gr_line (start 153.2001 64.2874) (end 135.4201 64.2874) (layer Edge.Cuts) (width 0.00254))
 (gr_line (start 153.2001 49.6824) (end 153.2001 64.2874) (layer Edge.Cuts) (width 0.00254))
 (gr_line (start 169.0751 49.6824) (end 153.2001 49.6824) (layer Edge.Cuts) (width 0.00254))
 (gr_line (start 169.0751 116.3574) (end 169.0751 49.6824) (layer Edge.Cuts) (width 0.00254))
 (gr_line (start 127.1651 129.0574) (end 156.3751 129.0574) (layer Edge.Cuts) (width 0.00254))
 (gr_line (start 114.4651 49.0474) (end 114.4651 116.3574) (layer Edge.Cuts) (width 0.00254))
 (segment (start 123.8631 117.6274) (end 123.3551 117.6274) (width 0.381) (layer B.Cu) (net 8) (status C00000))
 (segment (start 121.4501 92.8624) (end 118.9101 90.3224) (width 0.381) (layer B.Cu) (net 8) (status 800000))
 (segment (start 121.4501 115.7224) (end 121.4501 92.8624) (width 0.381) (layer B.Cu) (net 8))
 (segment (start 123.3551 117.6274) (end 121.4501 115.7224) (width 0.381) (layer B.Cu) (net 8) (status 400000))
 (segment (start 123.8631 121.4374) (end 122.0851 121.4374) (width 0.381) (layer B.Cu) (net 2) (status 400000))
 (segment (start 120.4341 94.3864) (end 118.9101 92.8624) (width 0.381) (layer B.Cu) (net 2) (status 800000))
 (segment (start 120.4341 119.7864) (end 120.4341 94.3864) (width 0.381) (layer B.Cu) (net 2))
 (segment (start 122.0851 121.4374) (end 120.4341 119.7864) (width 0.381) (layer B.Cu) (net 2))
 (segment (start 123.8631 120.1674) (end 124.8791 120.1674) (width 0.381) (layer B.Cu) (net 6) (status 400000))
 (segment (start 125.5141 120.8024) (end 125.5141 122.5804) (width 0.381) (layer B.Cu) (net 6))
 (segment (start 124.8791 120.1674) (end 125.5141 120.8024) (width 0.381) (layer B.Cu) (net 6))
 (segment (start 119.9261 122.5804) (end 118.9101 121.5644) (width 0.381) (layer B.Cu) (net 6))
 (segment (start 118.9101 121.5644) (end 118.9101 118.2624) (width 0.381) (layer B.Cu) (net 6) (status 800000))
 (segment (start 125.5141 122.5804) (end 119.9261 122.5804) (width 0.381) (layer B.Cu) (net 6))
 (segment (start 125.5141 122.5804) (end 125.5141 125.1689) (width 0.381) (layer B.Cu) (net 6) (status 800000))
 (segment (start 125.5141 125.1689) (end 125.5926 125.2474) (width 0.381) (layer B.Cu) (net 6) (status C00000))
 (segment (start 123.8631 118.8974) (end 124.6251 118.8974) (width 0.381) (layer B.Cu) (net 7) (status C00000))
 (segment (start 120.6881 64.9224) (end 118.9101 64.9224) (width 0.381) (layer B.Cu) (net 7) (status 800000))
 (segment (start 122.4661 66.7004) (end 120.6881 64.9224) (width 0.381) (layer B.Cu) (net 7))
 (segment (start 122.4661 113.4364) (end 122.4661 66.7004) (width 0.381) (layer B.Cu) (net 7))
 (segment (start 125.5141 116.4844) (end 122.4661 113.4364) (width 0.381) (layer B.Cu) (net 7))
 (segment (start 125.5141 118.0084) (end 125.5141 116.4844) (width 0.381) (layer B.Cu) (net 7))
 (segment (start 124.6251 118.8974) (end 125.5141 118.0084) (width 0.381) (layer B.Cu) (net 7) (status 400000))
 (segment (start 139.3571 114.4524) (end 139.7381 114.4524) (width 0.381) (layer B.Cu) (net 3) (status C00000))
 (segment (start 151.9301 114.4524) (end 154.5971 114.4524) (width 0.381) (layer B.Cu) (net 3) (status 800000))
 (segment (start 150.6601 115.7224) (end 151.9301 114.4524) (width 0.381) (layer B.Cu) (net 3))
 (segment (start 141.0081 115.7224) (end 150.6601 115.7224) (width 0.381) (layer B.Cu) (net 3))
 (segment (start 139.7381 114.4524) (end 141.0081 115.7224) (width 0.381) (layer B.Cu) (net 3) (status 400000))
 (segment (start 139.3571 114.4524) (end 128.8161 114.4524) (width 0.381) (layer B.Cu) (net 3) (status 400000))
 (segment (start 127.9271 120.1674) (end 129.1971 120.1674) (width 0.381) (layer B.Cu) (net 3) (status 800000))
 (segment (start 127.2921 119.5324) (end 127.9271 120.1674) (width 0.381) (layer B.Cu) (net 3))
 (segment (start 127.2921 115.9764) (end 127.2921 119.5324) (width 0.381) (layer B.Cu) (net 3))
 (segment (start 128.8161 114.4524) (end 127.2921 115.9764) (width 0.381) (layer B.Cu) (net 3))
 (segment (start 129.1971 118.8974) (end 133.0071 118.8974) (width 0.508) (layer B.Cu) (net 4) (status 400000))
 (segment (start 140.6271 116.9924) (end 140.5001 116.9924) (width 0.381) (layer B.Cu) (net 4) (status C00000))
 (segment (start 136.4361 115.4684) (end 133.0071 118.8974) (width 0.381) (layer B.Cu) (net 4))
 (segment (start 138.4681 115.4684) (end 136.4361 115.4684) (width 0.381) (layer B.Cu) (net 4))
 (segment (start 138.9761 115.9764) (end 138.4681 115.4684) (width 0.381) (layer B.Cu) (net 4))
 (segment (start 139.4841 115.9764) (end 138.9761 115.9764) (width 0.381) (layer B.Cu) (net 4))
 (segment (start 140.5001 116.9924) (end 139.4841 115.9764) (width 0.381) (layer B.Cu) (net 4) (status 400000))
 (segment (start 140.6271 116.9924) (end 151.1681 116.9924) (width 0.381) (layer B.Cu) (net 4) (status 400000))
 (segment (start 154.5971 115.7224) (end 155.8671 116.9924) (width 0.381) (layer B.Cu) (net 4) (status 800000))
 (segment (start 152.4381 115.7224) (end 154.5971 115.7224) (width 0.381) (layer B.Cu) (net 4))
 (segment (start 151.1681 116.9924) (end 152.4381 115.7224) (width 0.381) (layer B.Cu) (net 4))
 (segment (start 141.8971 114.4524) (end 149.8981 114.4524) (width 0.381) (layer B.Cu) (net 10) (status 400000))
 (segment (start 155.6131 112.9284) (end 157.1371 114.4524) (width 0.381) (layer B.Cu) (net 10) (status 800000))
 (segment (start 151.4221 112.9284) (end 155.6131 112.9284) (width 0.381) (layer B.Cu) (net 10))
 (segment (start 149.8981 114.4524) (end 151.4221 112.9284) (width 0.381) (layer B.Cu) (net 10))
 (segment (start 138.0871 116.9924) (end 138.0871 117.1194) (width 0.381) (layer B.Cu) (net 9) (status C00000))
 (segment (start 151.8031 118.5164) (end 153.3271 116.9924) (width 0.381) (layer B.Cu) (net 9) (status 800000))
 (segment (start 139.4841 118.5164) (end 151.8031 118.5164) (width 0.381) (layer B.Cu) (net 9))
 (segment (start 138.0871 117.1194) (end 139.4841 118.5164) (width 0.381) (layer B.Cu) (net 9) (status 400000))
 (segment (start 129.1971 121.4374) (end 129.1971 123.5179) (width 0.381) (layer B.Cu) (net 1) (status 400000))
 (segment (start 129.1971 123.5179) (end 127.4676 125.2474) (width 0.381) (layer B.Cu) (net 1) (status 800000)))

